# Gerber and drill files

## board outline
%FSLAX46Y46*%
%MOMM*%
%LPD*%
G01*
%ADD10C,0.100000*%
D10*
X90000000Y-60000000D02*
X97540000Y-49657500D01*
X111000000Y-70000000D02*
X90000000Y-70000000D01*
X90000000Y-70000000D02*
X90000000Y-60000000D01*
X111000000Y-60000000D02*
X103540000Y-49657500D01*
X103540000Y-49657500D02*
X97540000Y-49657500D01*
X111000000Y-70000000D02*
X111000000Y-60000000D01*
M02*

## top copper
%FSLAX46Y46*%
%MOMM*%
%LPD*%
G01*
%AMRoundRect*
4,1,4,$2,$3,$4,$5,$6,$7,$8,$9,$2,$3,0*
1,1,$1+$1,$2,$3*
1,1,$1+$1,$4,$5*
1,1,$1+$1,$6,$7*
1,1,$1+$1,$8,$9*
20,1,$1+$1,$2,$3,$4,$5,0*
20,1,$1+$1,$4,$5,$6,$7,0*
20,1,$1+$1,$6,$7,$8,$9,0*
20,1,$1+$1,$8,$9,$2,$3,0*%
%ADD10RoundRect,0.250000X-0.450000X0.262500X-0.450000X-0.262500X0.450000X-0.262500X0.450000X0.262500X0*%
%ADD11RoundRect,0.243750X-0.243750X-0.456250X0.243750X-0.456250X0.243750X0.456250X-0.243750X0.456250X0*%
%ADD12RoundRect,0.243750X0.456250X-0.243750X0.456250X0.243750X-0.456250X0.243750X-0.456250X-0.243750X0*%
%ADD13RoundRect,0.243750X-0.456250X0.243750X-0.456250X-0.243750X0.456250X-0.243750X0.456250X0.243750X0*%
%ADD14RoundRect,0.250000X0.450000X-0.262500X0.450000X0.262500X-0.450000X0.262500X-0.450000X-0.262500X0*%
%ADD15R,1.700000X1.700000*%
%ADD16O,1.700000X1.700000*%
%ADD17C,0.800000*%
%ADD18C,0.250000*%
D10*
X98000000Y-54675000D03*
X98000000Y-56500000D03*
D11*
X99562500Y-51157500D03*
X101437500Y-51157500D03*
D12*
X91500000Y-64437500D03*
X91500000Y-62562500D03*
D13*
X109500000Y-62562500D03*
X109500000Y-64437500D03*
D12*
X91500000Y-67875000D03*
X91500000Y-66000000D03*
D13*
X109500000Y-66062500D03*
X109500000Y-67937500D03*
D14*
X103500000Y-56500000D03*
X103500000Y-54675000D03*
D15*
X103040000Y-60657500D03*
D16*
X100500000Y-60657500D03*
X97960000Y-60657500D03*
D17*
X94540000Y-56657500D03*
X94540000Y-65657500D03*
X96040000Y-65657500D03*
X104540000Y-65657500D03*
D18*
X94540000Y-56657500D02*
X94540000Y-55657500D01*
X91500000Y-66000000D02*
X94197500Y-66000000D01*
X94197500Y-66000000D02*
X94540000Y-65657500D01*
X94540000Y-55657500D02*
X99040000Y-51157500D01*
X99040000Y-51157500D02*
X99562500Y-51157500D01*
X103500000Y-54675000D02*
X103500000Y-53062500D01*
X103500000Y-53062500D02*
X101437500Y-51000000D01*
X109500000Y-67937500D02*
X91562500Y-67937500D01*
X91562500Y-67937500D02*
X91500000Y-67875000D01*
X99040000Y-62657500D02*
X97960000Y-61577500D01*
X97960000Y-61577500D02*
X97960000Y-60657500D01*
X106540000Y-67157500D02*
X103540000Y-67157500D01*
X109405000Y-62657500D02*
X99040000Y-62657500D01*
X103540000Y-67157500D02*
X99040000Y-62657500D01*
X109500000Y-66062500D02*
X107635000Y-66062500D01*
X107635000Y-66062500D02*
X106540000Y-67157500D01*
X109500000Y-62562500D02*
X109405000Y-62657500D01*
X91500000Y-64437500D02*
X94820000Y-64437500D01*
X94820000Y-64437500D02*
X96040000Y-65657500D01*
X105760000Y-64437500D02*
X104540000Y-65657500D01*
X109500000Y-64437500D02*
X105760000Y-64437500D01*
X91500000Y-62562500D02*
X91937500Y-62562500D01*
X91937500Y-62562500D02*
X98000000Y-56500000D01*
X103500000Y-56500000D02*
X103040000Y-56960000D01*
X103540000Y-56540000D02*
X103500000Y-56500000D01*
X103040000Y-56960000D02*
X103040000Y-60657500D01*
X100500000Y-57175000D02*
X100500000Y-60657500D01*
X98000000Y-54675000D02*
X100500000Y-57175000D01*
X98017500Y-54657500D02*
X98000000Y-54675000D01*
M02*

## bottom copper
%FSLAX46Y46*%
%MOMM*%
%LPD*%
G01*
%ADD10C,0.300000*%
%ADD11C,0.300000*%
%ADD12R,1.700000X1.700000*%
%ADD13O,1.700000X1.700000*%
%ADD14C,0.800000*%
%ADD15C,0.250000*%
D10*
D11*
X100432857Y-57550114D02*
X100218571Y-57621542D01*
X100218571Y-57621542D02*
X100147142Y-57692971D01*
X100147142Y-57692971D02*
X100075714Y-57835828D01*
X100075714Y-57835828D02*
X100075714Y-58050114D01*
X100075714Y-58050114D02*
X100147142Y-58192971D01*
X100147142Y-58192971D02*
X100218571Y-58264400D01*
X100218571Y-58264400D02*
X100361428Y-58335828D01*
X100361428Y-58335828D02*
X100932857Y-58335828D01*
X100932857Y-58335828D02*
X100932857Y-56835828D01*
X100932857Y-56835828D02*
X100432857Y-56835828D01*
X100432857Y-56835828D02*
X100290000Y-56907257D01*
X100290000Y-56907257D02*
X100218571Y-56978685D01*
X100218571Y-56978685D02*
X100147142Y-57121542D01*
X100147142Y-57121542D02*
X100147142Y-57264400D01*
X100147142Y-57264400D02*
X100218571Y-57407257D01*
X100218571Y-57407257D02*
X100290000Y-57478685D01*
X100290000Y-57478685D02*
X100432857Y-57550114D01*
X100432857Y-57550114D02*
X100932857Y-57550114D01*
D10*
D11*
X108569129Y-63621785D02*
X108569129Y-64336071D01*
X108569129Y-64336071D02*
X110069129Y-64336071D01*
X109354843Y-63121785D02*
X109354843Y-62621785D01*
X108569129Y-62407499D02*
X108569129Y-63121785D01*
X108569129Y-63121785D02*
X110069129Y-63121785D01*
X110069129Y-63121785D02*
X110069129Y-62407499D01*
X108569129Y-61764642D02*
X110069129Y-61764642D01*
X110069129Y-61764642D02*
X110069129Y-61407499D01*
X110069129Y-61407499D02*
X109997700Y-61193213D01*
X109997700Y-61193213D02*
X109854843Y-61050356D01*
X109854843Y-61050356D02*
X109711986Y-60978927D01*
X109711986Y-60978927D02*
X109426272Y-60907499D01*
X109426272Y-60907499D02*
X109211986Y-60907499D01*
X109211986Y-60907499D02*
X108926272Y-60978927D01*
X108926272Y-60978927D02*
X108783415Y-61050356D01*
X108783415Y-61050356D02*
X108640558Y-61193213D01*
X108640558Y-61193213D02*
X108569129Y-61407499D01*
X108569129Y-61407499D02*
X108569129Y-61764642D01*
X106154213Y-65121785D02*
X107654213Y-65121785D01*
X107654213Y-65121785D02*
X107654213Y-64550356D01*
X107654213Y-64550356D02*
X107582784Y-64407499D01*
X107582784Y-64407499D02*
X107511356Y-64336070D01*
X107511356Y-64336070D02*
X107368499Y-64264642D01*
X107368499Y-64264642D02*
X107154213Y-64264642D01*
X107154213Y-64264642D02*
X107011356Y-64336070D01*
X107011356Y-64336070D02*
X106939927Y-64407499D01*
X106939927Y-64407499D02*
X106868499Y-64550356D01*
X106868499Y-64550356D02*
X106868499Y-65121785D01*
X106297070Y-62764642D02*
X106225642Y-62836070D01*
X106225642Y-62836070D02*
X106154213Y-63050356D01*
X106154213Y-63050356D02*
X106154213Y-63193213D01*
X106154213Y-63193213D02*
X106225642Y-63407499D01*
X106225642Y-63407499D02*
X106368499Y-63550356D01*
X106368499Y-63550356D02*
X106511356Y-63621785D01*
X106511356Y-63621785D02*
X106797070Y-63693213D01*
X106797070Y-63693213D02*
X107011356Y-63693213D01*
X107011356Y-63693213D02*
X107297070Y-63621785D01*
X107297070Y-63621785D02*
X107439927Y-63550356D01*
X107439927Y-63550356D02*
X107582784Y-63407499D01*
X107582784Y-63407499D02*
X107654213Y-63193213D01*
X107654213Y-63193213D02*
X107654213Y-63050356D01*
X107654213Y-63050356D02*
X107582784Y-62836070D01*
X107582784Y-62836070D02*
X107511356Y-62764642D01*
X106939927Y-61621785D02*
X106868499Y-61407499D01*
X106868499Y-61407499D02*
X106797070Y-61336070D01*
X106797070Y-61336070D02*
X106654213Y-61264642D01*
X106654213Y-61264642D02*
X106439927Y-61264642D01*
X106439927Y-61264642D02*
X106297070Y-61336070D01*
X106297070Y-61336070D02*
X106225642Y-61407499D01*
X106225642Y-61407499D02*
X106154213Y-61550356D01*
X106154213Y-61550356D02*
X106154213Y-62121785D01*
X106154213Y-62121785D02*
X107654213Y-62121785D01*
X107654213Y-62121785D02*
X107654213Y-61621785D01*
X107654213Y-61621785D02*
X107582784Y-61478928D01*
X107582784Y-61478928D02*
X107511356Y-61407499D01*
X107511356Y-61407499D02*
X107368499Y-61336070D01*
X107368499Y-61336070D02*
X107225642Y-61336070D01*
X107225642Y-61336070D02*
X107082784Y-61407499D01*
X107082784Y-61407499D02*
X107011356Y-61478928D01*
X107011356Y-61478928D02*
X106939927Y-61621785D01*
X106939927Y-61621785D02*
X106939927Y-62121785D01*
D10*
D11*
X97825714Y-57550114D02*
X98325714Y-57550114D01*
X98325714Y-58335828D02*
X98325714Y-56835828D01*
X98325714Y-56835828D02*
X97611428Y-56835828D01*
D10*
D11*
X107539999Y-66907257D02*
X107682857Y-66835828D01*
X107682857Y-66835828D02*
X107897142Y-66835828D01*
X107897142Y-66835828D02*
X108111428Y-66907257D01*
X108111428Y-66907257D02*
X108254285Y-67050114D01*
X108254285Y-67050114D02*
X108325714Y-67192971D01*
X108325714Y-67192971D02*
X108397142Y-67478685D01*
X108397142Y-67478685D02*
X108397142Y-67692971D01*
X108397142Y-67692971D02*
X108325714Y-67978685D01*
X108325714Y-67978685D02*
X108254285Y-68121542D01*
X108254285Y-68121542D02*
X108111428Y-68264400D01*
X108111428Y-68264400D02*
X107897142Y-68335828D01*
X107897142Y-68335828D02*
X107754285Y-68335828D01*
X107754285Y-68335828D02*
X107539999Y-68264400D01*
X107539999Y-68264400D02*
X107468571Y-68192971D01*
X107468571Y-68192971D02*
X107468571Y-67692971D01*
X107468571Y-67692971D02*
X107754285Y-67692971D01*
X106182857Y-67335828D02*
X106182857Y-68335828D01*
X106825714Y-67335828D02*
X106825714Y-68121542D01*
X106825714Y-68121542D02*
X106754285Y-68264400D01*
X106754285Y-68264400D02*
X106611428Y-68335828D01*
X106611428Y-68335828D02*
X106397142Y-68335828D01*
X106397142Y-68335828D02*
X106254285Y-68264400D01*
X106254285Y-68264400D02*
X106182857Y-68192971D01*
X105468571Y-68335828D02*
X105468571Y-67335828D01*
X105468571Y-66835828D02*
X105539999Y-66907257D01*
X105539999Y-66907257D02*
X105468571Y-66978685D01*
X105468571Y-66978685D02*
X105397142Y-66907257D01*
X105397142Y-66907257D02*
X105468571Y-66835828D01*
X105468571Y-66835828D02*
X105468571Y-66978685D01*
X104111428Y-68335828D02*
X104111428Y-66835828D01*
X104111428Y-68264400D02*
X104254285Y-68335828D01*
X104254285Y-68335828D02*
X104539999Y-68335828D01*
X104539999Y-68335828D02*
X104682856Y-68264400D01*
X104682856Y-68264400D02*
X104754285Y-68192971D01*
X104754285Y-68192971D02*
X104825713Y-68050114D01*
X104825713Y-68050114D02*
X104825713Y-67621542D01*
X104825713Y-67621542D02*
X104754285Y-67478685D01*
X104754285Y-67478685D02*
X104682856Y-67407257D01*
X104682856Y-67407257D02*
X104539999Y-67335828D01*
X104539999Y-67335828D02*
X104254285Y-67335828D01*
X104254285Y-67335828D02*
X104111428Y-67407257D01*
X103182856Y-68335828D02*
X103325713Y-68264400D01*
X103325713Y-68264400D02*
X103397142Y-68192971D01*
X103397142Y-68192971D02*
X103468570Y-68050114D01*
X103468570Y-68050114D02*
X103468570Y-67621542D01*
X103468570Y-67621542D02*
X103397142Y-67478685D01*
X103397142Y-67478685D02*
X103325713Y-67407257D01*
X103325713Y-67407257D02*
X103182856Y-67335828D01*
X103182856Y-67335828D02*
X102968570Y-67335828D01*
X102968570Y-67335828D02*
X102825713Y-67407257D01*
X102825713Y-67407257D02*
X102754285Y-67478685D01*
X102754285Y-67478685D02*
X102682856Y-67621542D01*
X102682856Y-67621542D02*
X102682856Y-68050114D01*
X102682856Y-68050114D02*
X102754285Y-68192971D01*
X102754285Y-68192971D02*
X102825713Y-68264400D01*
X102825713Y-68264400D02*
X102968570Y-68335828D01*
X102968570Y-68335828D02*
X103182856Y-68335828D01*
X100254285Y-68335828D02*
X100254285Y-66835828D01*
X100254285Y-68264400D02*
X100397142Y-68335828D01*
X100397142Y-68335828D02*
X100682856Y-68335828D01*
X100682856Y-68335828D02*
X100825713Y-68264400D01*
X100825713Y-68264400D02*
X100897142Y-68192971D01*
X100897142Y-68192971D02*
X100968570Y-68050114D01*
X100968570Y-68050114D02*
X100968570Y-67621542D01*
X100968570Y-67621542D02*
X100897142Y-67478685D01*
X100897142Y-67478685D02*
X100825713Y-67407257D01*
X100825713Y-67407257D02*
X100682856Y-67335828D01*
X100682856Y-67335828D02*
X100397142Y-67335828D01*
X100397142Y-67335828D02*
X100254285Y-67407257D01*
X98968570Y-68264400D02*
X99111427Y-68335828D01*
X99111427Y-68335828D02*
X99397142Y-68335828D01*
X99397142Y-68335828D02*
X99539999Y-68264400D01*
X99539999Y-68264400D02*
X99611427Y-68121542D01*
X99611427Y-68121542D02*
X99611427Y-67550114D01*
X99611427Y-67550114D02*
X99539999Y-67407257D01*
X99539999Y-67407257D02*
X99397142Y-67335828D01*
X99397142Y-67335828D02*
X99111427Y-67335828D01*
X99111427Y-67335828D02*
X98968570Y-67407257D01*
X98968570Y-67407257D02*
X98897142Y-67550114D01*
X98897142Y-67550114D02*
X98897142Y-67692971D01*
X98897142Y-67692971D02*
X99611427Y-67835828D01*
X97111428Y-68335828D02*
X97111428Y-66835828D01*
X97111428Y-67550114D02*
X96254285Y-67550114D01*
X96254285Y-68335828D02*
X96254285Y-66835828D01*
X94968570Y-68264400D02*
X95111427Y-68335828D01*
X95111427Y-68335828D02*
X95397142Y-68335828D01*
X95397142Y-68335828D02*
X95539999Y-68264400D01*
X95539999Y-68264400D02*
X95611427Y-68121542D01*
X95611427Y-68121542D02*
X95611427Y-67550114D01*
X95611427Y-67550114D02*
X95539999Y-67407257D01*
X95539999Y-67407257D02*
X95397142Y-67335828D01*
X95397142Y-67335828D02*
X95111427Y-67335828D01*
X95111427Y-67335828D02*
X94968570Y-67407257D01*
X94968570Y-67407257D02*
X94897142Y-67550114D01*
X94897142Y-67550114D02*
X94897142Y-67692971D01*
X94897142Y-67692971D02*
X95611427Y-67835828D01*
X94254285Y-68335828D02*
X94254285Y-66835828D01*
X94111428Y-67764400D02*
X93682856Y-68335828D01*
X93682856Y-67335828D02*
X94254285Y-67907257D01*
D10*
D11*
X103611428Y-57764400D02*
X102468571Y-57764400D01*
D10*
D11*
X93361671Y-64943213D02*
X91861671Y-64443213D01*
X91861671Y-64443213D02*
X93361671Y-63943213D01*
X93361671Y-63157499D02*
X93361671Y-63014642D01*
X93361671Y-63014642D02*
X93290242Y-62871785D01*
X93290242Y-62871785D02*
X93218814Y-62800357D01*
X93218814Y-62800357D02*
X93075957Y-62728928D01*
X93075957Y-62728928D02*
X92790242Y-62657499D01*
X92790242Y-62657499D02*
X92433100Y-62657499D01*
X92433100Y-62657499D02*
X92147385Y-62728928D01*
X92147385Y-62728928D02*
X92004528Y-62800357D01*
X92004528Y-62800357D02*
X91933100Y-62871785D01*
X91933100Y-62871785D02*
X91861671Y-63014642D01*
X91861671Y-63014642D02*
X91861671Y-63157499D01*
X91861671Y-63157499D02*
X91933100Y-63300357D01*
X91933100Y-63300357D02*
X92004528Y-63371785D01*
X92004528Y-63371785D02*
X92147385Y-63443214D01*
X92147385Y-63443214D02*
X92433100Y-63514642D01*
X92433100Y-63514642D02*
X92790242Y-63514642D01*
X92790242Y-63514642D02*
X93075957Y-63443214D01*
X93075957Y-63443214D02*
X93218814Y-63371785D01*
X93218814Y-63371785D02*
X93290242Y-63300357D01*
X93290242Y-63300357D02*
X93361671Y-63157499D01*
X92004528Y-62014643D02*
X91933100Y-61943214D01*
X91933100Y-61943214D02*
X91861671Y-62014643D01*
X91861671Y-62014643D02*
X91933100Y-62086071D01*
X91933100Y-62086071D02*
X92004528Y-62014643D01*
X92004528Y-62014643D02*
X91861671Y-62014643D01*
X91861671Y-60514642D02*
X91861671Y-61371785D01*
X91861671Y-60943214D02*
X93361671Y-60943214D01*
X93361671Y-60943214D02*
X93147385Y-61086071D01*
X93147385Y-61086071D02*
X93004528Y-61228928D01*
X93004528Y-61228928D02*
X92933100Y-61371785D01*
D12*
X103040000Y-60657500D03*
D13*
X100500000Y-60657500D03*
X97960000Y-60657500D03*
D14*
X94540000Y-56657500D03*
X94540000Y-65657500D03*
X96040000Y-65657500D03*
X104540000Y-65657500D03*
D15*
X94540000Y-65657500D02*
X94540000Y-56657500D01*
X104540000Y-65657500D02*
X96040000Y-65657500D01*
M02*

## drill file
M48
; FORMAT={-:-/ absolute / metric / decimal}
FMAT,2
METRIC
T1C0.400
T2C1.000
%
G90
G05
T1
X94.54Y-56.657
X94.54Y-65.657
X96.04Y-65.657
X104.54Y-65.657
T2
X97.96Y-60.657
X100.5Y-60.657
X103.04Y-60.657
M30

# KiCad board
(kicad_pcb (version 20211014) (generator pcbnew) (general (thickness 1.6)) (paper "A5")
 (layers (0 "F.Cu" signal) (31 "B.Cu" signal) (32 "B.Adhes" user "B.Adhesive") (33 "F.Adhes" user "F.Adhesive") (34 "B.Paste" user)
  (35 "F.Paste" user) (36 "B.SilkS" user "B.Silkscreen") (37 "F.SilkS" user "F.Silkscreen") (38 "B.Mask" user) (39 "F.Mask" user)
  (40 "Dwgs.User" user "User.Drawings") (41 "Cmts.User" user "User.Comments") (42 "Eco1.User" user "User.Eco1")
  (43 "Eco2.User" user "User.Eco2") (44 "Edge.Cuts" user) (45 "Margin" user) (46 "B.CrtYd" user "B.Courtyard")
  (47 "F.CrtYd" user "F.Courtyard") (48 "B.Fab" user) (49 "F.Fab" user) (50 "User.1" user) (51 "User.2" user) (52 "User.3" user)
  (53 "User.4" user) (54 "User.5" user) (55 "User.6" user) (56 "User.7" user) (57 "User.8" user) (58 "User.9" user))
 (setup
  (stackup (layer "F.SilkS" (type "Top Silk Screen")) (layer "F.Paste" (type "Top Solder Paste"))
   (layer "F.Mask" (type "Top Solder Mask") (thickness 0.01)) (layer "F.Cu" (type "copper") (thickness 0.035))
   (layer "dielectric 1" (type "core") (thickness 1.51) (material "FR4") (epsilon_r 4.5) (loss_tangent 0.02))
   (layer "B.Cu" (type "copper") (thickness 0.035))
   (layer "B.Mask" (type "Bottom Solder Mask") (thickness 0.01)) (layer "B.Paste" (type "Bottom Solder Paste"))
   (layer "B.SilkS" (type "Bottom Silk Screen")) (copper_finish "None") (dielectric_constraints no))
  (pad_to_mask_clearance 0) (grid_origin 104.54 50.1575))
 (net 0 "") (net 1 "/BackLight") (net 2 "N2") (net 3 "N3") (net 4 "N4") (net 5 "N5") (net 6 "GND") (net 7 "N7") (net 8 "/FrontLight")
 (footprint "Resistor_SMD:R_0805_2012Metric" (layer "F.Cu") (at 98 55.5875 -90)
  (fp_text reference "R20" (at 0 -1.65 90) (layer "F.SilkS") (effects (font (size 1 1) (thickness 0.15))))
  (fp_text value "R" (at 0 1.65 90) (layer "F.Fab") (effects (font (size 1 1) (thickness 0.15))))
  (pad "1" smd roundrect locked (at -0.9125 0 270) (size 1.025 1.4) (layers "F.Cu" "F.Paste" "F.Mask") (roundrect_rratio 0.243902)
   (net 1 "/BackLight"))
  (pad "2" smd roundrect locked (at 0.9125 0 270) (size 1.025 1.4) (layers "F.Cu" "F.Paste" "F.Mask") (roundrect_rratio 0.243902)
   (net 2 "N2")))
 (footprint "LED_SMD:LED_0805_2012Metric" (layer "F.Cu") (at 100.5 51.1575)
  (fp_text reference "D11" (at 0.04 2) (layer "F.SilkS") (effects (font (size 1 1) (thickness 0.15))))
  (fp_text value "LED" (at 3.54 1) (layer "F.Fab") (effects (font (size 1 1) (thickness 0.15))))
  (pad "1" smd roundrect locked (at -0.9375 0) (size 0.975 1.4) (layers "F.Cu" "F.Paste" "F.Mask") (roundrect_rratio 0.25) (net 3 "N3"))
  (pad "2" smd roundrect locked (at 0.9375 0) (size 0.975 1.4) (layers "F.Cu" "F.Paste" "F.Mask") (roundrect_rratio 0.25) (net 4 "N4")))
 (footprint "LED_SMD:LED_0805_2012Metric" (layer "F.Cu") (at 91.5 63.5 90)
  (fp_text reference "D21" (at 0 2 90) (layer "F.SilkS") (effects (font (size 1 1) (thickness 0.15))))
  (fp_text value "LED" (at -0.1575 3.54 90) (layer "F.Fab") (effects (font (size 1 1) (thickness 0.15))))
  (pad "1" smd roundrect locked (at -0.9375 0 90) (size 0.975 1.4) (layers "F.Cu" "F.Paste" "F.Mask") (roundrect_rratio 0.25) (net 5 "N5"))
  (pad "2" smd roundrect locked (at 0.9375 0 90) (size 0.975 1.4) (layers "F.Cu" "F.Paste" "F.Mask") (roundrect_rratio 0.25) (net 2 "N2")))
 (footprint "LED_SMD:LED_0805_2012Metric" (layer "F.Cu") (at 109.5 63.5 -90)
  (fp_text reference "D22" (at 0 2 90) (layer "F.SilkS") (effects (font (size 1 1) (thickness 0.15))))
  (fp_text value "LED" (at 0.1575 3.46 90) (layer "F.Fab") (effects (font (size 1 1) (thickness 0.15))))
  (pad "1" smd roundrect locked (at -0.9375 0 270) (size 0.975 1.4) (layers "F.Cu" "F.Paste" "F.Mask") (roundrect_rratio 0.25) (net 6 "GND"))
  (pad "2" smd roundrect locked (at 0.9375 0 270) (size 0.975 1.4) (layers "F.Cu" "F.Paste" "F.Mask") (roundrect_rratio 0.25) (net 5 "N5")))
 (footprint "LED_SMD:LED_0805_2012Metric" (layer "F.Cu") (at 91.5 66.9375 90)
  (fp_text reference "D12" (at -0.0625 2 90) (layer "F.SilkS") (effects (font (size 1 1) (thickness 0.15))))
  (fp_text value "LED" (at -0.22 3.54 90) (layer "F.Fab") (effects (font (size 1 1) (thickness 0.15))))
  (pad "1" smd roundrect locked (at -0.9375 0 90) (size 0.975 1.4) (layers "F.Cu" "F.Paste" "F.Mask") (roundrect_rratio 0.25) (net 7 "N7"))
  (pad "2" smd roundrect locked (at 0.9375 0 90) (size 0.975 1.4) (layers "F.Cu" "F.Paste" "F.Mask") (roundrect_rratio 0.25) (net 3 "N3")))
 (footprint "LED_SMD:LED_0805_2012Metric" (layer "F.Cu") (at 109.5 67 -90)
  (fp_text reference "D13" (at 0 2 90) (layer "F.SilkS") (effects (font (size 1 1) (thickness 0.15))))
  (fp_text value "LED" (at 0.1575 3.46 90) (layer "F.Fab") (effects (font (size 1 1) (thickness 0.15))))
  (pad "1" smd roundrect locked (at -0.9375 0 270) (size 0.975 1.4) (layers "F.Cu" "F.Paste" "F.Mask") (roundrect_rratio 0.25) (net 6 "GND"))
  (pad "2" smd roundrect locked (at 0.9375 0 270) (size 0.975 1.4) (layers "F.Cu" "F.Paste" "F.Mask") (roundrect_rratio 0.25) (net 7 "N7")))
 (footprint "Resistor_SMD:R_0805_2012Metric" (layer "F.Cu") (at 103.5 55.5875 90)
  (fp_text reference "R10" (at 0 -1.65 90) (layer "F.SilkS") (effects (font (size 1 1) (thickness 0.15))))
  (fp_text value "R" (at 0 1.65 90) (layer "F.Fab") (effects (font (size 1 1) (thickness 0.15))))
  (pad "1" smd roundrect locked (at -0.9125 0 90) (size 1.025 1.4) (layers "F.Cu" "F.Paste" "F.Mask") (roundrect_rratio 0.243902)
   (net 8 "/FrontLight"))
  (pad "2" smd roundrect locked (at 0.9125 0 90) (size 1.025 1.4) (layers "F.Cu" "F.Paste" "F.Mask") (roundrect_rratio 0.243902)
   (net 4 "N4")))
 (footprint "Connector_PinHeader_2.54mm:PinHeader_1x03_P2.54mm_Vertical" (layer "B.Cu") (at 103.04 60.6575 90)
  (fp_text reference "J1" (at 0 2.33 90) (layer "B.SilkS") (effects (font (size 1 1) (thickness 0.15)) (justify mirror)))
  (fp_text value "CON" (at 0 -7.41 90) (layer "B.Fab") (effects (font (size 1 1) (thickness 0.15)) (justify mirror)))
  (pad "1" thru_hole rect locked (at 0 0 90) (size 1.7 1.7) (drill 1) (layers *.Cu *.Mask) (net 8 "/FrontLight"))
  (pad "2" thru_hole oval locked (at 0 -2.54 90) (size 1.7 1.7) (drill 1) (layers *.Cu *.Mask) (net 1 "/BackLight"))
  (pad "3" thru_hole oval locked (at 0 -5.08 90) (size 1.7 1.7) (drill 1) (layers *.Cu *.Mask) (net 6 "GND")))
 (gr_line (start 90 60) (end 97.54 49.6575) (layer "Edge.Cuts") (width 0.1))
 (gr_line (start 111 70) (end 90 70) (layer "Edge.Cuts") (width 0.1))
 (gr_line (start 90 70) (end 90 60) (layer "Edge.Cuts") (width 0.1))
 (gr_line (start 111 60) (end 103.54 49.6575) (layer "Edge.Cuts") (width 0.1))
 (gr_line (start 103.54 49.6575) (end 97.54 49.6575) (layer "Edge.Cuts") (width 0.1))
 (gr_line (start 111 70) (end 111 60) (layer "Edge.Cuts") (width 0.1))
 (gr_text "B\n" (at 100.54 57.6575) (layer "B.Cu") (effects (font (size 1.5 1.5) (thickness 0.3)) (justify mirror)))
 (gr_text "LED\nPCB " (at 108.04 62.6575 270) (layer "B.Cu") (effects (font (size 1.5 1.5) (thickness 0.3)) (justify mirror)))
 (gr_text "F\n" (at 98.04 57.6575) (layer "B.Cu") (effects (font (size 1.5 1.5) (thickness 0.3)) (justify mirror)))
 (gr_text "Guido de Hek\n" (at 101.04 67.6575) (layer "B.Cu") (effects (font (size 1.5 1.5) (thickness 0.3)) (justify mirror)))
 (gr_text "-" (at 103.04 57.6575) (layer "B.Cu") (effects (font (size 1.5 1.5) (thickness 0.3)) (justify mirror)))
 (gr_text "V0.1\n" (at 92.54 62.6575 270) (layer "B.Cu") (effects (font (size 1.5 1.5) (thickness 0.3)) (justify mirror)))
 (segment (start 94.54 56.6575) (end 94.54 55.6575) (width 0.25) (layer "F.Cu") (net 3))
 (segment (start 91.5 66) (end 94.1975 66) (width 0.25) (layer "F.Cu") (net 3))
 (segment (start 94.1975 66) (end 94.54 65.6575) (width 0.25) (layer "F.Cu") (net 3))
 (segment (start 94.54 55.6575) (end 99.04 51.1575) (width 0.25) (layer "F.Cu") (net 3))
 (segment (start 99.04 51.1575) (end 99.5625 51.1575) (width 0.25) (layer "F.Cu") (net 3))
 (via (at 94.54 56.6575) (size 0.8) (drill 0.4) (layers "F.Cu" "B.Cu") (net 3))
 (via (at 94.54 65.6575) (size 0.8) (drill 0.4) (layers "F.Cu" "B.Cu") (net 3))
 (segment (start 94.54 65.6575) (end 94.54 56.6575) (width 0.25) (layer "B.Cu") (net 3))
 (segment (start 103.5 54.675) (end 103.5 53.0625) (width 0.25) (layer "F.Cu") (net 4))
 (segment (start 103.5 53.0625) (end 101.4375 51) (width 0.25) (layer "F.Cu") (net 4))
 (segment (start 109.5 67.9375) (end 91.5625 67.9375) (width 0.25) (layer "F.Cu") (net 7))
 (segment (start 91.5625 67.9375) (end 91.5 67.875) (width 0.25) (layer "F.Cu") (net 7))
 (segment (start 99.04 62.6575) (end 97.96 61.5775) (width 0.25) (layer "F.Cu") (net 6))
 (segment (start 97.96 61.5775) (end 97.96 60.6575) (width 0.25) (layer "F.Cu") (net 6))
 (segment (start 106.54 67.1575) (end 103.54 67.1575) (width 0.25) (layer "F.Cu") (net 6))
 (segment (start 109.405 62.6575) (end 99.04 62.6575) (width 0.25) (layer "F.Cu") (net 6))
 (segment (start 103.54 67.1575) (end 99.04 62.6575) (width 0.25) (layer "F.Cu") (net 6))
 (segment (start 109.5 66.0625) (end 107.635 66.0625) (width 0.25) (layer "F.Cu") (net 6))
 (segment (start 107.635 66.0625) (end 106.54 67.1575) (width 0.25) (layer "F.Cu") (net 6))
 (segment (start 109.5 62.5625) (end 109.405 62.6575) (width 0.25) (layer "F.Cu") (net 6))
 (segment (start 91.5 64.4375) (end 94.82 64.4375) (width 0.25) (layer "F.Cu") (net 5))
 (segment (start 94.82 64.4375) (end 96.04 65.6575) (width 0.25) (layer "F.Cu") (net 5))
 (segment (start 105.76 64.4375) (end 104.54 65.6575) (width 0.25) (layer "F.Cu") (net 5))
 (segment (start 109.5 64.4375) (end 105.76 64.4375) (width 0.25) (layer "F.Cu") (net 5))
 (via (at 96.04 65.6575) (size 0.8) (drill 0.4) (layers "F.Cu" "B.Cu") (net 5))
 (via (at 104.54 65.6575) (size 0.8) (drill 0.4) (layers "F.Cu" "B.Cu") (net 5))
 (segment (start 104.54 65.6575) (end 96.04 65.6575) (width 0.25) (layer "B.Cu") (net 5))
 (segment (start 91.5 62.5625) (end 91.9375 62.5625) (width 0.25) (layer "F.Cu") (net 2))
 (segment (start 91.9375 62.5625) (end 98 56.5) (width 0.25) (layer "F.Cu") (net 2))
 (segment (start 103.5 56.5) (end 103.04 56.96) (width 0.25) (layer "F.Cu") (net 8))
 (segment (start 103.54 56.54) (end 103.5 56.5) (width 0.25) (layer "F.Cu") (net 8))
 (segment (start 103.04 56.96) (end 103.04 60.6575) (width 0.25) (layer "F.Cu") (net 8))
 (segment (start 100.5 57.175) (end 100.5 60.6575) (width 0.25) (layer "F.Cu") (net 1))
 (segment (start 98 54.675) (end 100.5 57.175) (width 0.25) (layer "F.Cu") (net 1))
 (segment (start 98.0175 54.6575) (end 98 54.675) (width 0.25) (layer "F.Cu") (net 1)))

